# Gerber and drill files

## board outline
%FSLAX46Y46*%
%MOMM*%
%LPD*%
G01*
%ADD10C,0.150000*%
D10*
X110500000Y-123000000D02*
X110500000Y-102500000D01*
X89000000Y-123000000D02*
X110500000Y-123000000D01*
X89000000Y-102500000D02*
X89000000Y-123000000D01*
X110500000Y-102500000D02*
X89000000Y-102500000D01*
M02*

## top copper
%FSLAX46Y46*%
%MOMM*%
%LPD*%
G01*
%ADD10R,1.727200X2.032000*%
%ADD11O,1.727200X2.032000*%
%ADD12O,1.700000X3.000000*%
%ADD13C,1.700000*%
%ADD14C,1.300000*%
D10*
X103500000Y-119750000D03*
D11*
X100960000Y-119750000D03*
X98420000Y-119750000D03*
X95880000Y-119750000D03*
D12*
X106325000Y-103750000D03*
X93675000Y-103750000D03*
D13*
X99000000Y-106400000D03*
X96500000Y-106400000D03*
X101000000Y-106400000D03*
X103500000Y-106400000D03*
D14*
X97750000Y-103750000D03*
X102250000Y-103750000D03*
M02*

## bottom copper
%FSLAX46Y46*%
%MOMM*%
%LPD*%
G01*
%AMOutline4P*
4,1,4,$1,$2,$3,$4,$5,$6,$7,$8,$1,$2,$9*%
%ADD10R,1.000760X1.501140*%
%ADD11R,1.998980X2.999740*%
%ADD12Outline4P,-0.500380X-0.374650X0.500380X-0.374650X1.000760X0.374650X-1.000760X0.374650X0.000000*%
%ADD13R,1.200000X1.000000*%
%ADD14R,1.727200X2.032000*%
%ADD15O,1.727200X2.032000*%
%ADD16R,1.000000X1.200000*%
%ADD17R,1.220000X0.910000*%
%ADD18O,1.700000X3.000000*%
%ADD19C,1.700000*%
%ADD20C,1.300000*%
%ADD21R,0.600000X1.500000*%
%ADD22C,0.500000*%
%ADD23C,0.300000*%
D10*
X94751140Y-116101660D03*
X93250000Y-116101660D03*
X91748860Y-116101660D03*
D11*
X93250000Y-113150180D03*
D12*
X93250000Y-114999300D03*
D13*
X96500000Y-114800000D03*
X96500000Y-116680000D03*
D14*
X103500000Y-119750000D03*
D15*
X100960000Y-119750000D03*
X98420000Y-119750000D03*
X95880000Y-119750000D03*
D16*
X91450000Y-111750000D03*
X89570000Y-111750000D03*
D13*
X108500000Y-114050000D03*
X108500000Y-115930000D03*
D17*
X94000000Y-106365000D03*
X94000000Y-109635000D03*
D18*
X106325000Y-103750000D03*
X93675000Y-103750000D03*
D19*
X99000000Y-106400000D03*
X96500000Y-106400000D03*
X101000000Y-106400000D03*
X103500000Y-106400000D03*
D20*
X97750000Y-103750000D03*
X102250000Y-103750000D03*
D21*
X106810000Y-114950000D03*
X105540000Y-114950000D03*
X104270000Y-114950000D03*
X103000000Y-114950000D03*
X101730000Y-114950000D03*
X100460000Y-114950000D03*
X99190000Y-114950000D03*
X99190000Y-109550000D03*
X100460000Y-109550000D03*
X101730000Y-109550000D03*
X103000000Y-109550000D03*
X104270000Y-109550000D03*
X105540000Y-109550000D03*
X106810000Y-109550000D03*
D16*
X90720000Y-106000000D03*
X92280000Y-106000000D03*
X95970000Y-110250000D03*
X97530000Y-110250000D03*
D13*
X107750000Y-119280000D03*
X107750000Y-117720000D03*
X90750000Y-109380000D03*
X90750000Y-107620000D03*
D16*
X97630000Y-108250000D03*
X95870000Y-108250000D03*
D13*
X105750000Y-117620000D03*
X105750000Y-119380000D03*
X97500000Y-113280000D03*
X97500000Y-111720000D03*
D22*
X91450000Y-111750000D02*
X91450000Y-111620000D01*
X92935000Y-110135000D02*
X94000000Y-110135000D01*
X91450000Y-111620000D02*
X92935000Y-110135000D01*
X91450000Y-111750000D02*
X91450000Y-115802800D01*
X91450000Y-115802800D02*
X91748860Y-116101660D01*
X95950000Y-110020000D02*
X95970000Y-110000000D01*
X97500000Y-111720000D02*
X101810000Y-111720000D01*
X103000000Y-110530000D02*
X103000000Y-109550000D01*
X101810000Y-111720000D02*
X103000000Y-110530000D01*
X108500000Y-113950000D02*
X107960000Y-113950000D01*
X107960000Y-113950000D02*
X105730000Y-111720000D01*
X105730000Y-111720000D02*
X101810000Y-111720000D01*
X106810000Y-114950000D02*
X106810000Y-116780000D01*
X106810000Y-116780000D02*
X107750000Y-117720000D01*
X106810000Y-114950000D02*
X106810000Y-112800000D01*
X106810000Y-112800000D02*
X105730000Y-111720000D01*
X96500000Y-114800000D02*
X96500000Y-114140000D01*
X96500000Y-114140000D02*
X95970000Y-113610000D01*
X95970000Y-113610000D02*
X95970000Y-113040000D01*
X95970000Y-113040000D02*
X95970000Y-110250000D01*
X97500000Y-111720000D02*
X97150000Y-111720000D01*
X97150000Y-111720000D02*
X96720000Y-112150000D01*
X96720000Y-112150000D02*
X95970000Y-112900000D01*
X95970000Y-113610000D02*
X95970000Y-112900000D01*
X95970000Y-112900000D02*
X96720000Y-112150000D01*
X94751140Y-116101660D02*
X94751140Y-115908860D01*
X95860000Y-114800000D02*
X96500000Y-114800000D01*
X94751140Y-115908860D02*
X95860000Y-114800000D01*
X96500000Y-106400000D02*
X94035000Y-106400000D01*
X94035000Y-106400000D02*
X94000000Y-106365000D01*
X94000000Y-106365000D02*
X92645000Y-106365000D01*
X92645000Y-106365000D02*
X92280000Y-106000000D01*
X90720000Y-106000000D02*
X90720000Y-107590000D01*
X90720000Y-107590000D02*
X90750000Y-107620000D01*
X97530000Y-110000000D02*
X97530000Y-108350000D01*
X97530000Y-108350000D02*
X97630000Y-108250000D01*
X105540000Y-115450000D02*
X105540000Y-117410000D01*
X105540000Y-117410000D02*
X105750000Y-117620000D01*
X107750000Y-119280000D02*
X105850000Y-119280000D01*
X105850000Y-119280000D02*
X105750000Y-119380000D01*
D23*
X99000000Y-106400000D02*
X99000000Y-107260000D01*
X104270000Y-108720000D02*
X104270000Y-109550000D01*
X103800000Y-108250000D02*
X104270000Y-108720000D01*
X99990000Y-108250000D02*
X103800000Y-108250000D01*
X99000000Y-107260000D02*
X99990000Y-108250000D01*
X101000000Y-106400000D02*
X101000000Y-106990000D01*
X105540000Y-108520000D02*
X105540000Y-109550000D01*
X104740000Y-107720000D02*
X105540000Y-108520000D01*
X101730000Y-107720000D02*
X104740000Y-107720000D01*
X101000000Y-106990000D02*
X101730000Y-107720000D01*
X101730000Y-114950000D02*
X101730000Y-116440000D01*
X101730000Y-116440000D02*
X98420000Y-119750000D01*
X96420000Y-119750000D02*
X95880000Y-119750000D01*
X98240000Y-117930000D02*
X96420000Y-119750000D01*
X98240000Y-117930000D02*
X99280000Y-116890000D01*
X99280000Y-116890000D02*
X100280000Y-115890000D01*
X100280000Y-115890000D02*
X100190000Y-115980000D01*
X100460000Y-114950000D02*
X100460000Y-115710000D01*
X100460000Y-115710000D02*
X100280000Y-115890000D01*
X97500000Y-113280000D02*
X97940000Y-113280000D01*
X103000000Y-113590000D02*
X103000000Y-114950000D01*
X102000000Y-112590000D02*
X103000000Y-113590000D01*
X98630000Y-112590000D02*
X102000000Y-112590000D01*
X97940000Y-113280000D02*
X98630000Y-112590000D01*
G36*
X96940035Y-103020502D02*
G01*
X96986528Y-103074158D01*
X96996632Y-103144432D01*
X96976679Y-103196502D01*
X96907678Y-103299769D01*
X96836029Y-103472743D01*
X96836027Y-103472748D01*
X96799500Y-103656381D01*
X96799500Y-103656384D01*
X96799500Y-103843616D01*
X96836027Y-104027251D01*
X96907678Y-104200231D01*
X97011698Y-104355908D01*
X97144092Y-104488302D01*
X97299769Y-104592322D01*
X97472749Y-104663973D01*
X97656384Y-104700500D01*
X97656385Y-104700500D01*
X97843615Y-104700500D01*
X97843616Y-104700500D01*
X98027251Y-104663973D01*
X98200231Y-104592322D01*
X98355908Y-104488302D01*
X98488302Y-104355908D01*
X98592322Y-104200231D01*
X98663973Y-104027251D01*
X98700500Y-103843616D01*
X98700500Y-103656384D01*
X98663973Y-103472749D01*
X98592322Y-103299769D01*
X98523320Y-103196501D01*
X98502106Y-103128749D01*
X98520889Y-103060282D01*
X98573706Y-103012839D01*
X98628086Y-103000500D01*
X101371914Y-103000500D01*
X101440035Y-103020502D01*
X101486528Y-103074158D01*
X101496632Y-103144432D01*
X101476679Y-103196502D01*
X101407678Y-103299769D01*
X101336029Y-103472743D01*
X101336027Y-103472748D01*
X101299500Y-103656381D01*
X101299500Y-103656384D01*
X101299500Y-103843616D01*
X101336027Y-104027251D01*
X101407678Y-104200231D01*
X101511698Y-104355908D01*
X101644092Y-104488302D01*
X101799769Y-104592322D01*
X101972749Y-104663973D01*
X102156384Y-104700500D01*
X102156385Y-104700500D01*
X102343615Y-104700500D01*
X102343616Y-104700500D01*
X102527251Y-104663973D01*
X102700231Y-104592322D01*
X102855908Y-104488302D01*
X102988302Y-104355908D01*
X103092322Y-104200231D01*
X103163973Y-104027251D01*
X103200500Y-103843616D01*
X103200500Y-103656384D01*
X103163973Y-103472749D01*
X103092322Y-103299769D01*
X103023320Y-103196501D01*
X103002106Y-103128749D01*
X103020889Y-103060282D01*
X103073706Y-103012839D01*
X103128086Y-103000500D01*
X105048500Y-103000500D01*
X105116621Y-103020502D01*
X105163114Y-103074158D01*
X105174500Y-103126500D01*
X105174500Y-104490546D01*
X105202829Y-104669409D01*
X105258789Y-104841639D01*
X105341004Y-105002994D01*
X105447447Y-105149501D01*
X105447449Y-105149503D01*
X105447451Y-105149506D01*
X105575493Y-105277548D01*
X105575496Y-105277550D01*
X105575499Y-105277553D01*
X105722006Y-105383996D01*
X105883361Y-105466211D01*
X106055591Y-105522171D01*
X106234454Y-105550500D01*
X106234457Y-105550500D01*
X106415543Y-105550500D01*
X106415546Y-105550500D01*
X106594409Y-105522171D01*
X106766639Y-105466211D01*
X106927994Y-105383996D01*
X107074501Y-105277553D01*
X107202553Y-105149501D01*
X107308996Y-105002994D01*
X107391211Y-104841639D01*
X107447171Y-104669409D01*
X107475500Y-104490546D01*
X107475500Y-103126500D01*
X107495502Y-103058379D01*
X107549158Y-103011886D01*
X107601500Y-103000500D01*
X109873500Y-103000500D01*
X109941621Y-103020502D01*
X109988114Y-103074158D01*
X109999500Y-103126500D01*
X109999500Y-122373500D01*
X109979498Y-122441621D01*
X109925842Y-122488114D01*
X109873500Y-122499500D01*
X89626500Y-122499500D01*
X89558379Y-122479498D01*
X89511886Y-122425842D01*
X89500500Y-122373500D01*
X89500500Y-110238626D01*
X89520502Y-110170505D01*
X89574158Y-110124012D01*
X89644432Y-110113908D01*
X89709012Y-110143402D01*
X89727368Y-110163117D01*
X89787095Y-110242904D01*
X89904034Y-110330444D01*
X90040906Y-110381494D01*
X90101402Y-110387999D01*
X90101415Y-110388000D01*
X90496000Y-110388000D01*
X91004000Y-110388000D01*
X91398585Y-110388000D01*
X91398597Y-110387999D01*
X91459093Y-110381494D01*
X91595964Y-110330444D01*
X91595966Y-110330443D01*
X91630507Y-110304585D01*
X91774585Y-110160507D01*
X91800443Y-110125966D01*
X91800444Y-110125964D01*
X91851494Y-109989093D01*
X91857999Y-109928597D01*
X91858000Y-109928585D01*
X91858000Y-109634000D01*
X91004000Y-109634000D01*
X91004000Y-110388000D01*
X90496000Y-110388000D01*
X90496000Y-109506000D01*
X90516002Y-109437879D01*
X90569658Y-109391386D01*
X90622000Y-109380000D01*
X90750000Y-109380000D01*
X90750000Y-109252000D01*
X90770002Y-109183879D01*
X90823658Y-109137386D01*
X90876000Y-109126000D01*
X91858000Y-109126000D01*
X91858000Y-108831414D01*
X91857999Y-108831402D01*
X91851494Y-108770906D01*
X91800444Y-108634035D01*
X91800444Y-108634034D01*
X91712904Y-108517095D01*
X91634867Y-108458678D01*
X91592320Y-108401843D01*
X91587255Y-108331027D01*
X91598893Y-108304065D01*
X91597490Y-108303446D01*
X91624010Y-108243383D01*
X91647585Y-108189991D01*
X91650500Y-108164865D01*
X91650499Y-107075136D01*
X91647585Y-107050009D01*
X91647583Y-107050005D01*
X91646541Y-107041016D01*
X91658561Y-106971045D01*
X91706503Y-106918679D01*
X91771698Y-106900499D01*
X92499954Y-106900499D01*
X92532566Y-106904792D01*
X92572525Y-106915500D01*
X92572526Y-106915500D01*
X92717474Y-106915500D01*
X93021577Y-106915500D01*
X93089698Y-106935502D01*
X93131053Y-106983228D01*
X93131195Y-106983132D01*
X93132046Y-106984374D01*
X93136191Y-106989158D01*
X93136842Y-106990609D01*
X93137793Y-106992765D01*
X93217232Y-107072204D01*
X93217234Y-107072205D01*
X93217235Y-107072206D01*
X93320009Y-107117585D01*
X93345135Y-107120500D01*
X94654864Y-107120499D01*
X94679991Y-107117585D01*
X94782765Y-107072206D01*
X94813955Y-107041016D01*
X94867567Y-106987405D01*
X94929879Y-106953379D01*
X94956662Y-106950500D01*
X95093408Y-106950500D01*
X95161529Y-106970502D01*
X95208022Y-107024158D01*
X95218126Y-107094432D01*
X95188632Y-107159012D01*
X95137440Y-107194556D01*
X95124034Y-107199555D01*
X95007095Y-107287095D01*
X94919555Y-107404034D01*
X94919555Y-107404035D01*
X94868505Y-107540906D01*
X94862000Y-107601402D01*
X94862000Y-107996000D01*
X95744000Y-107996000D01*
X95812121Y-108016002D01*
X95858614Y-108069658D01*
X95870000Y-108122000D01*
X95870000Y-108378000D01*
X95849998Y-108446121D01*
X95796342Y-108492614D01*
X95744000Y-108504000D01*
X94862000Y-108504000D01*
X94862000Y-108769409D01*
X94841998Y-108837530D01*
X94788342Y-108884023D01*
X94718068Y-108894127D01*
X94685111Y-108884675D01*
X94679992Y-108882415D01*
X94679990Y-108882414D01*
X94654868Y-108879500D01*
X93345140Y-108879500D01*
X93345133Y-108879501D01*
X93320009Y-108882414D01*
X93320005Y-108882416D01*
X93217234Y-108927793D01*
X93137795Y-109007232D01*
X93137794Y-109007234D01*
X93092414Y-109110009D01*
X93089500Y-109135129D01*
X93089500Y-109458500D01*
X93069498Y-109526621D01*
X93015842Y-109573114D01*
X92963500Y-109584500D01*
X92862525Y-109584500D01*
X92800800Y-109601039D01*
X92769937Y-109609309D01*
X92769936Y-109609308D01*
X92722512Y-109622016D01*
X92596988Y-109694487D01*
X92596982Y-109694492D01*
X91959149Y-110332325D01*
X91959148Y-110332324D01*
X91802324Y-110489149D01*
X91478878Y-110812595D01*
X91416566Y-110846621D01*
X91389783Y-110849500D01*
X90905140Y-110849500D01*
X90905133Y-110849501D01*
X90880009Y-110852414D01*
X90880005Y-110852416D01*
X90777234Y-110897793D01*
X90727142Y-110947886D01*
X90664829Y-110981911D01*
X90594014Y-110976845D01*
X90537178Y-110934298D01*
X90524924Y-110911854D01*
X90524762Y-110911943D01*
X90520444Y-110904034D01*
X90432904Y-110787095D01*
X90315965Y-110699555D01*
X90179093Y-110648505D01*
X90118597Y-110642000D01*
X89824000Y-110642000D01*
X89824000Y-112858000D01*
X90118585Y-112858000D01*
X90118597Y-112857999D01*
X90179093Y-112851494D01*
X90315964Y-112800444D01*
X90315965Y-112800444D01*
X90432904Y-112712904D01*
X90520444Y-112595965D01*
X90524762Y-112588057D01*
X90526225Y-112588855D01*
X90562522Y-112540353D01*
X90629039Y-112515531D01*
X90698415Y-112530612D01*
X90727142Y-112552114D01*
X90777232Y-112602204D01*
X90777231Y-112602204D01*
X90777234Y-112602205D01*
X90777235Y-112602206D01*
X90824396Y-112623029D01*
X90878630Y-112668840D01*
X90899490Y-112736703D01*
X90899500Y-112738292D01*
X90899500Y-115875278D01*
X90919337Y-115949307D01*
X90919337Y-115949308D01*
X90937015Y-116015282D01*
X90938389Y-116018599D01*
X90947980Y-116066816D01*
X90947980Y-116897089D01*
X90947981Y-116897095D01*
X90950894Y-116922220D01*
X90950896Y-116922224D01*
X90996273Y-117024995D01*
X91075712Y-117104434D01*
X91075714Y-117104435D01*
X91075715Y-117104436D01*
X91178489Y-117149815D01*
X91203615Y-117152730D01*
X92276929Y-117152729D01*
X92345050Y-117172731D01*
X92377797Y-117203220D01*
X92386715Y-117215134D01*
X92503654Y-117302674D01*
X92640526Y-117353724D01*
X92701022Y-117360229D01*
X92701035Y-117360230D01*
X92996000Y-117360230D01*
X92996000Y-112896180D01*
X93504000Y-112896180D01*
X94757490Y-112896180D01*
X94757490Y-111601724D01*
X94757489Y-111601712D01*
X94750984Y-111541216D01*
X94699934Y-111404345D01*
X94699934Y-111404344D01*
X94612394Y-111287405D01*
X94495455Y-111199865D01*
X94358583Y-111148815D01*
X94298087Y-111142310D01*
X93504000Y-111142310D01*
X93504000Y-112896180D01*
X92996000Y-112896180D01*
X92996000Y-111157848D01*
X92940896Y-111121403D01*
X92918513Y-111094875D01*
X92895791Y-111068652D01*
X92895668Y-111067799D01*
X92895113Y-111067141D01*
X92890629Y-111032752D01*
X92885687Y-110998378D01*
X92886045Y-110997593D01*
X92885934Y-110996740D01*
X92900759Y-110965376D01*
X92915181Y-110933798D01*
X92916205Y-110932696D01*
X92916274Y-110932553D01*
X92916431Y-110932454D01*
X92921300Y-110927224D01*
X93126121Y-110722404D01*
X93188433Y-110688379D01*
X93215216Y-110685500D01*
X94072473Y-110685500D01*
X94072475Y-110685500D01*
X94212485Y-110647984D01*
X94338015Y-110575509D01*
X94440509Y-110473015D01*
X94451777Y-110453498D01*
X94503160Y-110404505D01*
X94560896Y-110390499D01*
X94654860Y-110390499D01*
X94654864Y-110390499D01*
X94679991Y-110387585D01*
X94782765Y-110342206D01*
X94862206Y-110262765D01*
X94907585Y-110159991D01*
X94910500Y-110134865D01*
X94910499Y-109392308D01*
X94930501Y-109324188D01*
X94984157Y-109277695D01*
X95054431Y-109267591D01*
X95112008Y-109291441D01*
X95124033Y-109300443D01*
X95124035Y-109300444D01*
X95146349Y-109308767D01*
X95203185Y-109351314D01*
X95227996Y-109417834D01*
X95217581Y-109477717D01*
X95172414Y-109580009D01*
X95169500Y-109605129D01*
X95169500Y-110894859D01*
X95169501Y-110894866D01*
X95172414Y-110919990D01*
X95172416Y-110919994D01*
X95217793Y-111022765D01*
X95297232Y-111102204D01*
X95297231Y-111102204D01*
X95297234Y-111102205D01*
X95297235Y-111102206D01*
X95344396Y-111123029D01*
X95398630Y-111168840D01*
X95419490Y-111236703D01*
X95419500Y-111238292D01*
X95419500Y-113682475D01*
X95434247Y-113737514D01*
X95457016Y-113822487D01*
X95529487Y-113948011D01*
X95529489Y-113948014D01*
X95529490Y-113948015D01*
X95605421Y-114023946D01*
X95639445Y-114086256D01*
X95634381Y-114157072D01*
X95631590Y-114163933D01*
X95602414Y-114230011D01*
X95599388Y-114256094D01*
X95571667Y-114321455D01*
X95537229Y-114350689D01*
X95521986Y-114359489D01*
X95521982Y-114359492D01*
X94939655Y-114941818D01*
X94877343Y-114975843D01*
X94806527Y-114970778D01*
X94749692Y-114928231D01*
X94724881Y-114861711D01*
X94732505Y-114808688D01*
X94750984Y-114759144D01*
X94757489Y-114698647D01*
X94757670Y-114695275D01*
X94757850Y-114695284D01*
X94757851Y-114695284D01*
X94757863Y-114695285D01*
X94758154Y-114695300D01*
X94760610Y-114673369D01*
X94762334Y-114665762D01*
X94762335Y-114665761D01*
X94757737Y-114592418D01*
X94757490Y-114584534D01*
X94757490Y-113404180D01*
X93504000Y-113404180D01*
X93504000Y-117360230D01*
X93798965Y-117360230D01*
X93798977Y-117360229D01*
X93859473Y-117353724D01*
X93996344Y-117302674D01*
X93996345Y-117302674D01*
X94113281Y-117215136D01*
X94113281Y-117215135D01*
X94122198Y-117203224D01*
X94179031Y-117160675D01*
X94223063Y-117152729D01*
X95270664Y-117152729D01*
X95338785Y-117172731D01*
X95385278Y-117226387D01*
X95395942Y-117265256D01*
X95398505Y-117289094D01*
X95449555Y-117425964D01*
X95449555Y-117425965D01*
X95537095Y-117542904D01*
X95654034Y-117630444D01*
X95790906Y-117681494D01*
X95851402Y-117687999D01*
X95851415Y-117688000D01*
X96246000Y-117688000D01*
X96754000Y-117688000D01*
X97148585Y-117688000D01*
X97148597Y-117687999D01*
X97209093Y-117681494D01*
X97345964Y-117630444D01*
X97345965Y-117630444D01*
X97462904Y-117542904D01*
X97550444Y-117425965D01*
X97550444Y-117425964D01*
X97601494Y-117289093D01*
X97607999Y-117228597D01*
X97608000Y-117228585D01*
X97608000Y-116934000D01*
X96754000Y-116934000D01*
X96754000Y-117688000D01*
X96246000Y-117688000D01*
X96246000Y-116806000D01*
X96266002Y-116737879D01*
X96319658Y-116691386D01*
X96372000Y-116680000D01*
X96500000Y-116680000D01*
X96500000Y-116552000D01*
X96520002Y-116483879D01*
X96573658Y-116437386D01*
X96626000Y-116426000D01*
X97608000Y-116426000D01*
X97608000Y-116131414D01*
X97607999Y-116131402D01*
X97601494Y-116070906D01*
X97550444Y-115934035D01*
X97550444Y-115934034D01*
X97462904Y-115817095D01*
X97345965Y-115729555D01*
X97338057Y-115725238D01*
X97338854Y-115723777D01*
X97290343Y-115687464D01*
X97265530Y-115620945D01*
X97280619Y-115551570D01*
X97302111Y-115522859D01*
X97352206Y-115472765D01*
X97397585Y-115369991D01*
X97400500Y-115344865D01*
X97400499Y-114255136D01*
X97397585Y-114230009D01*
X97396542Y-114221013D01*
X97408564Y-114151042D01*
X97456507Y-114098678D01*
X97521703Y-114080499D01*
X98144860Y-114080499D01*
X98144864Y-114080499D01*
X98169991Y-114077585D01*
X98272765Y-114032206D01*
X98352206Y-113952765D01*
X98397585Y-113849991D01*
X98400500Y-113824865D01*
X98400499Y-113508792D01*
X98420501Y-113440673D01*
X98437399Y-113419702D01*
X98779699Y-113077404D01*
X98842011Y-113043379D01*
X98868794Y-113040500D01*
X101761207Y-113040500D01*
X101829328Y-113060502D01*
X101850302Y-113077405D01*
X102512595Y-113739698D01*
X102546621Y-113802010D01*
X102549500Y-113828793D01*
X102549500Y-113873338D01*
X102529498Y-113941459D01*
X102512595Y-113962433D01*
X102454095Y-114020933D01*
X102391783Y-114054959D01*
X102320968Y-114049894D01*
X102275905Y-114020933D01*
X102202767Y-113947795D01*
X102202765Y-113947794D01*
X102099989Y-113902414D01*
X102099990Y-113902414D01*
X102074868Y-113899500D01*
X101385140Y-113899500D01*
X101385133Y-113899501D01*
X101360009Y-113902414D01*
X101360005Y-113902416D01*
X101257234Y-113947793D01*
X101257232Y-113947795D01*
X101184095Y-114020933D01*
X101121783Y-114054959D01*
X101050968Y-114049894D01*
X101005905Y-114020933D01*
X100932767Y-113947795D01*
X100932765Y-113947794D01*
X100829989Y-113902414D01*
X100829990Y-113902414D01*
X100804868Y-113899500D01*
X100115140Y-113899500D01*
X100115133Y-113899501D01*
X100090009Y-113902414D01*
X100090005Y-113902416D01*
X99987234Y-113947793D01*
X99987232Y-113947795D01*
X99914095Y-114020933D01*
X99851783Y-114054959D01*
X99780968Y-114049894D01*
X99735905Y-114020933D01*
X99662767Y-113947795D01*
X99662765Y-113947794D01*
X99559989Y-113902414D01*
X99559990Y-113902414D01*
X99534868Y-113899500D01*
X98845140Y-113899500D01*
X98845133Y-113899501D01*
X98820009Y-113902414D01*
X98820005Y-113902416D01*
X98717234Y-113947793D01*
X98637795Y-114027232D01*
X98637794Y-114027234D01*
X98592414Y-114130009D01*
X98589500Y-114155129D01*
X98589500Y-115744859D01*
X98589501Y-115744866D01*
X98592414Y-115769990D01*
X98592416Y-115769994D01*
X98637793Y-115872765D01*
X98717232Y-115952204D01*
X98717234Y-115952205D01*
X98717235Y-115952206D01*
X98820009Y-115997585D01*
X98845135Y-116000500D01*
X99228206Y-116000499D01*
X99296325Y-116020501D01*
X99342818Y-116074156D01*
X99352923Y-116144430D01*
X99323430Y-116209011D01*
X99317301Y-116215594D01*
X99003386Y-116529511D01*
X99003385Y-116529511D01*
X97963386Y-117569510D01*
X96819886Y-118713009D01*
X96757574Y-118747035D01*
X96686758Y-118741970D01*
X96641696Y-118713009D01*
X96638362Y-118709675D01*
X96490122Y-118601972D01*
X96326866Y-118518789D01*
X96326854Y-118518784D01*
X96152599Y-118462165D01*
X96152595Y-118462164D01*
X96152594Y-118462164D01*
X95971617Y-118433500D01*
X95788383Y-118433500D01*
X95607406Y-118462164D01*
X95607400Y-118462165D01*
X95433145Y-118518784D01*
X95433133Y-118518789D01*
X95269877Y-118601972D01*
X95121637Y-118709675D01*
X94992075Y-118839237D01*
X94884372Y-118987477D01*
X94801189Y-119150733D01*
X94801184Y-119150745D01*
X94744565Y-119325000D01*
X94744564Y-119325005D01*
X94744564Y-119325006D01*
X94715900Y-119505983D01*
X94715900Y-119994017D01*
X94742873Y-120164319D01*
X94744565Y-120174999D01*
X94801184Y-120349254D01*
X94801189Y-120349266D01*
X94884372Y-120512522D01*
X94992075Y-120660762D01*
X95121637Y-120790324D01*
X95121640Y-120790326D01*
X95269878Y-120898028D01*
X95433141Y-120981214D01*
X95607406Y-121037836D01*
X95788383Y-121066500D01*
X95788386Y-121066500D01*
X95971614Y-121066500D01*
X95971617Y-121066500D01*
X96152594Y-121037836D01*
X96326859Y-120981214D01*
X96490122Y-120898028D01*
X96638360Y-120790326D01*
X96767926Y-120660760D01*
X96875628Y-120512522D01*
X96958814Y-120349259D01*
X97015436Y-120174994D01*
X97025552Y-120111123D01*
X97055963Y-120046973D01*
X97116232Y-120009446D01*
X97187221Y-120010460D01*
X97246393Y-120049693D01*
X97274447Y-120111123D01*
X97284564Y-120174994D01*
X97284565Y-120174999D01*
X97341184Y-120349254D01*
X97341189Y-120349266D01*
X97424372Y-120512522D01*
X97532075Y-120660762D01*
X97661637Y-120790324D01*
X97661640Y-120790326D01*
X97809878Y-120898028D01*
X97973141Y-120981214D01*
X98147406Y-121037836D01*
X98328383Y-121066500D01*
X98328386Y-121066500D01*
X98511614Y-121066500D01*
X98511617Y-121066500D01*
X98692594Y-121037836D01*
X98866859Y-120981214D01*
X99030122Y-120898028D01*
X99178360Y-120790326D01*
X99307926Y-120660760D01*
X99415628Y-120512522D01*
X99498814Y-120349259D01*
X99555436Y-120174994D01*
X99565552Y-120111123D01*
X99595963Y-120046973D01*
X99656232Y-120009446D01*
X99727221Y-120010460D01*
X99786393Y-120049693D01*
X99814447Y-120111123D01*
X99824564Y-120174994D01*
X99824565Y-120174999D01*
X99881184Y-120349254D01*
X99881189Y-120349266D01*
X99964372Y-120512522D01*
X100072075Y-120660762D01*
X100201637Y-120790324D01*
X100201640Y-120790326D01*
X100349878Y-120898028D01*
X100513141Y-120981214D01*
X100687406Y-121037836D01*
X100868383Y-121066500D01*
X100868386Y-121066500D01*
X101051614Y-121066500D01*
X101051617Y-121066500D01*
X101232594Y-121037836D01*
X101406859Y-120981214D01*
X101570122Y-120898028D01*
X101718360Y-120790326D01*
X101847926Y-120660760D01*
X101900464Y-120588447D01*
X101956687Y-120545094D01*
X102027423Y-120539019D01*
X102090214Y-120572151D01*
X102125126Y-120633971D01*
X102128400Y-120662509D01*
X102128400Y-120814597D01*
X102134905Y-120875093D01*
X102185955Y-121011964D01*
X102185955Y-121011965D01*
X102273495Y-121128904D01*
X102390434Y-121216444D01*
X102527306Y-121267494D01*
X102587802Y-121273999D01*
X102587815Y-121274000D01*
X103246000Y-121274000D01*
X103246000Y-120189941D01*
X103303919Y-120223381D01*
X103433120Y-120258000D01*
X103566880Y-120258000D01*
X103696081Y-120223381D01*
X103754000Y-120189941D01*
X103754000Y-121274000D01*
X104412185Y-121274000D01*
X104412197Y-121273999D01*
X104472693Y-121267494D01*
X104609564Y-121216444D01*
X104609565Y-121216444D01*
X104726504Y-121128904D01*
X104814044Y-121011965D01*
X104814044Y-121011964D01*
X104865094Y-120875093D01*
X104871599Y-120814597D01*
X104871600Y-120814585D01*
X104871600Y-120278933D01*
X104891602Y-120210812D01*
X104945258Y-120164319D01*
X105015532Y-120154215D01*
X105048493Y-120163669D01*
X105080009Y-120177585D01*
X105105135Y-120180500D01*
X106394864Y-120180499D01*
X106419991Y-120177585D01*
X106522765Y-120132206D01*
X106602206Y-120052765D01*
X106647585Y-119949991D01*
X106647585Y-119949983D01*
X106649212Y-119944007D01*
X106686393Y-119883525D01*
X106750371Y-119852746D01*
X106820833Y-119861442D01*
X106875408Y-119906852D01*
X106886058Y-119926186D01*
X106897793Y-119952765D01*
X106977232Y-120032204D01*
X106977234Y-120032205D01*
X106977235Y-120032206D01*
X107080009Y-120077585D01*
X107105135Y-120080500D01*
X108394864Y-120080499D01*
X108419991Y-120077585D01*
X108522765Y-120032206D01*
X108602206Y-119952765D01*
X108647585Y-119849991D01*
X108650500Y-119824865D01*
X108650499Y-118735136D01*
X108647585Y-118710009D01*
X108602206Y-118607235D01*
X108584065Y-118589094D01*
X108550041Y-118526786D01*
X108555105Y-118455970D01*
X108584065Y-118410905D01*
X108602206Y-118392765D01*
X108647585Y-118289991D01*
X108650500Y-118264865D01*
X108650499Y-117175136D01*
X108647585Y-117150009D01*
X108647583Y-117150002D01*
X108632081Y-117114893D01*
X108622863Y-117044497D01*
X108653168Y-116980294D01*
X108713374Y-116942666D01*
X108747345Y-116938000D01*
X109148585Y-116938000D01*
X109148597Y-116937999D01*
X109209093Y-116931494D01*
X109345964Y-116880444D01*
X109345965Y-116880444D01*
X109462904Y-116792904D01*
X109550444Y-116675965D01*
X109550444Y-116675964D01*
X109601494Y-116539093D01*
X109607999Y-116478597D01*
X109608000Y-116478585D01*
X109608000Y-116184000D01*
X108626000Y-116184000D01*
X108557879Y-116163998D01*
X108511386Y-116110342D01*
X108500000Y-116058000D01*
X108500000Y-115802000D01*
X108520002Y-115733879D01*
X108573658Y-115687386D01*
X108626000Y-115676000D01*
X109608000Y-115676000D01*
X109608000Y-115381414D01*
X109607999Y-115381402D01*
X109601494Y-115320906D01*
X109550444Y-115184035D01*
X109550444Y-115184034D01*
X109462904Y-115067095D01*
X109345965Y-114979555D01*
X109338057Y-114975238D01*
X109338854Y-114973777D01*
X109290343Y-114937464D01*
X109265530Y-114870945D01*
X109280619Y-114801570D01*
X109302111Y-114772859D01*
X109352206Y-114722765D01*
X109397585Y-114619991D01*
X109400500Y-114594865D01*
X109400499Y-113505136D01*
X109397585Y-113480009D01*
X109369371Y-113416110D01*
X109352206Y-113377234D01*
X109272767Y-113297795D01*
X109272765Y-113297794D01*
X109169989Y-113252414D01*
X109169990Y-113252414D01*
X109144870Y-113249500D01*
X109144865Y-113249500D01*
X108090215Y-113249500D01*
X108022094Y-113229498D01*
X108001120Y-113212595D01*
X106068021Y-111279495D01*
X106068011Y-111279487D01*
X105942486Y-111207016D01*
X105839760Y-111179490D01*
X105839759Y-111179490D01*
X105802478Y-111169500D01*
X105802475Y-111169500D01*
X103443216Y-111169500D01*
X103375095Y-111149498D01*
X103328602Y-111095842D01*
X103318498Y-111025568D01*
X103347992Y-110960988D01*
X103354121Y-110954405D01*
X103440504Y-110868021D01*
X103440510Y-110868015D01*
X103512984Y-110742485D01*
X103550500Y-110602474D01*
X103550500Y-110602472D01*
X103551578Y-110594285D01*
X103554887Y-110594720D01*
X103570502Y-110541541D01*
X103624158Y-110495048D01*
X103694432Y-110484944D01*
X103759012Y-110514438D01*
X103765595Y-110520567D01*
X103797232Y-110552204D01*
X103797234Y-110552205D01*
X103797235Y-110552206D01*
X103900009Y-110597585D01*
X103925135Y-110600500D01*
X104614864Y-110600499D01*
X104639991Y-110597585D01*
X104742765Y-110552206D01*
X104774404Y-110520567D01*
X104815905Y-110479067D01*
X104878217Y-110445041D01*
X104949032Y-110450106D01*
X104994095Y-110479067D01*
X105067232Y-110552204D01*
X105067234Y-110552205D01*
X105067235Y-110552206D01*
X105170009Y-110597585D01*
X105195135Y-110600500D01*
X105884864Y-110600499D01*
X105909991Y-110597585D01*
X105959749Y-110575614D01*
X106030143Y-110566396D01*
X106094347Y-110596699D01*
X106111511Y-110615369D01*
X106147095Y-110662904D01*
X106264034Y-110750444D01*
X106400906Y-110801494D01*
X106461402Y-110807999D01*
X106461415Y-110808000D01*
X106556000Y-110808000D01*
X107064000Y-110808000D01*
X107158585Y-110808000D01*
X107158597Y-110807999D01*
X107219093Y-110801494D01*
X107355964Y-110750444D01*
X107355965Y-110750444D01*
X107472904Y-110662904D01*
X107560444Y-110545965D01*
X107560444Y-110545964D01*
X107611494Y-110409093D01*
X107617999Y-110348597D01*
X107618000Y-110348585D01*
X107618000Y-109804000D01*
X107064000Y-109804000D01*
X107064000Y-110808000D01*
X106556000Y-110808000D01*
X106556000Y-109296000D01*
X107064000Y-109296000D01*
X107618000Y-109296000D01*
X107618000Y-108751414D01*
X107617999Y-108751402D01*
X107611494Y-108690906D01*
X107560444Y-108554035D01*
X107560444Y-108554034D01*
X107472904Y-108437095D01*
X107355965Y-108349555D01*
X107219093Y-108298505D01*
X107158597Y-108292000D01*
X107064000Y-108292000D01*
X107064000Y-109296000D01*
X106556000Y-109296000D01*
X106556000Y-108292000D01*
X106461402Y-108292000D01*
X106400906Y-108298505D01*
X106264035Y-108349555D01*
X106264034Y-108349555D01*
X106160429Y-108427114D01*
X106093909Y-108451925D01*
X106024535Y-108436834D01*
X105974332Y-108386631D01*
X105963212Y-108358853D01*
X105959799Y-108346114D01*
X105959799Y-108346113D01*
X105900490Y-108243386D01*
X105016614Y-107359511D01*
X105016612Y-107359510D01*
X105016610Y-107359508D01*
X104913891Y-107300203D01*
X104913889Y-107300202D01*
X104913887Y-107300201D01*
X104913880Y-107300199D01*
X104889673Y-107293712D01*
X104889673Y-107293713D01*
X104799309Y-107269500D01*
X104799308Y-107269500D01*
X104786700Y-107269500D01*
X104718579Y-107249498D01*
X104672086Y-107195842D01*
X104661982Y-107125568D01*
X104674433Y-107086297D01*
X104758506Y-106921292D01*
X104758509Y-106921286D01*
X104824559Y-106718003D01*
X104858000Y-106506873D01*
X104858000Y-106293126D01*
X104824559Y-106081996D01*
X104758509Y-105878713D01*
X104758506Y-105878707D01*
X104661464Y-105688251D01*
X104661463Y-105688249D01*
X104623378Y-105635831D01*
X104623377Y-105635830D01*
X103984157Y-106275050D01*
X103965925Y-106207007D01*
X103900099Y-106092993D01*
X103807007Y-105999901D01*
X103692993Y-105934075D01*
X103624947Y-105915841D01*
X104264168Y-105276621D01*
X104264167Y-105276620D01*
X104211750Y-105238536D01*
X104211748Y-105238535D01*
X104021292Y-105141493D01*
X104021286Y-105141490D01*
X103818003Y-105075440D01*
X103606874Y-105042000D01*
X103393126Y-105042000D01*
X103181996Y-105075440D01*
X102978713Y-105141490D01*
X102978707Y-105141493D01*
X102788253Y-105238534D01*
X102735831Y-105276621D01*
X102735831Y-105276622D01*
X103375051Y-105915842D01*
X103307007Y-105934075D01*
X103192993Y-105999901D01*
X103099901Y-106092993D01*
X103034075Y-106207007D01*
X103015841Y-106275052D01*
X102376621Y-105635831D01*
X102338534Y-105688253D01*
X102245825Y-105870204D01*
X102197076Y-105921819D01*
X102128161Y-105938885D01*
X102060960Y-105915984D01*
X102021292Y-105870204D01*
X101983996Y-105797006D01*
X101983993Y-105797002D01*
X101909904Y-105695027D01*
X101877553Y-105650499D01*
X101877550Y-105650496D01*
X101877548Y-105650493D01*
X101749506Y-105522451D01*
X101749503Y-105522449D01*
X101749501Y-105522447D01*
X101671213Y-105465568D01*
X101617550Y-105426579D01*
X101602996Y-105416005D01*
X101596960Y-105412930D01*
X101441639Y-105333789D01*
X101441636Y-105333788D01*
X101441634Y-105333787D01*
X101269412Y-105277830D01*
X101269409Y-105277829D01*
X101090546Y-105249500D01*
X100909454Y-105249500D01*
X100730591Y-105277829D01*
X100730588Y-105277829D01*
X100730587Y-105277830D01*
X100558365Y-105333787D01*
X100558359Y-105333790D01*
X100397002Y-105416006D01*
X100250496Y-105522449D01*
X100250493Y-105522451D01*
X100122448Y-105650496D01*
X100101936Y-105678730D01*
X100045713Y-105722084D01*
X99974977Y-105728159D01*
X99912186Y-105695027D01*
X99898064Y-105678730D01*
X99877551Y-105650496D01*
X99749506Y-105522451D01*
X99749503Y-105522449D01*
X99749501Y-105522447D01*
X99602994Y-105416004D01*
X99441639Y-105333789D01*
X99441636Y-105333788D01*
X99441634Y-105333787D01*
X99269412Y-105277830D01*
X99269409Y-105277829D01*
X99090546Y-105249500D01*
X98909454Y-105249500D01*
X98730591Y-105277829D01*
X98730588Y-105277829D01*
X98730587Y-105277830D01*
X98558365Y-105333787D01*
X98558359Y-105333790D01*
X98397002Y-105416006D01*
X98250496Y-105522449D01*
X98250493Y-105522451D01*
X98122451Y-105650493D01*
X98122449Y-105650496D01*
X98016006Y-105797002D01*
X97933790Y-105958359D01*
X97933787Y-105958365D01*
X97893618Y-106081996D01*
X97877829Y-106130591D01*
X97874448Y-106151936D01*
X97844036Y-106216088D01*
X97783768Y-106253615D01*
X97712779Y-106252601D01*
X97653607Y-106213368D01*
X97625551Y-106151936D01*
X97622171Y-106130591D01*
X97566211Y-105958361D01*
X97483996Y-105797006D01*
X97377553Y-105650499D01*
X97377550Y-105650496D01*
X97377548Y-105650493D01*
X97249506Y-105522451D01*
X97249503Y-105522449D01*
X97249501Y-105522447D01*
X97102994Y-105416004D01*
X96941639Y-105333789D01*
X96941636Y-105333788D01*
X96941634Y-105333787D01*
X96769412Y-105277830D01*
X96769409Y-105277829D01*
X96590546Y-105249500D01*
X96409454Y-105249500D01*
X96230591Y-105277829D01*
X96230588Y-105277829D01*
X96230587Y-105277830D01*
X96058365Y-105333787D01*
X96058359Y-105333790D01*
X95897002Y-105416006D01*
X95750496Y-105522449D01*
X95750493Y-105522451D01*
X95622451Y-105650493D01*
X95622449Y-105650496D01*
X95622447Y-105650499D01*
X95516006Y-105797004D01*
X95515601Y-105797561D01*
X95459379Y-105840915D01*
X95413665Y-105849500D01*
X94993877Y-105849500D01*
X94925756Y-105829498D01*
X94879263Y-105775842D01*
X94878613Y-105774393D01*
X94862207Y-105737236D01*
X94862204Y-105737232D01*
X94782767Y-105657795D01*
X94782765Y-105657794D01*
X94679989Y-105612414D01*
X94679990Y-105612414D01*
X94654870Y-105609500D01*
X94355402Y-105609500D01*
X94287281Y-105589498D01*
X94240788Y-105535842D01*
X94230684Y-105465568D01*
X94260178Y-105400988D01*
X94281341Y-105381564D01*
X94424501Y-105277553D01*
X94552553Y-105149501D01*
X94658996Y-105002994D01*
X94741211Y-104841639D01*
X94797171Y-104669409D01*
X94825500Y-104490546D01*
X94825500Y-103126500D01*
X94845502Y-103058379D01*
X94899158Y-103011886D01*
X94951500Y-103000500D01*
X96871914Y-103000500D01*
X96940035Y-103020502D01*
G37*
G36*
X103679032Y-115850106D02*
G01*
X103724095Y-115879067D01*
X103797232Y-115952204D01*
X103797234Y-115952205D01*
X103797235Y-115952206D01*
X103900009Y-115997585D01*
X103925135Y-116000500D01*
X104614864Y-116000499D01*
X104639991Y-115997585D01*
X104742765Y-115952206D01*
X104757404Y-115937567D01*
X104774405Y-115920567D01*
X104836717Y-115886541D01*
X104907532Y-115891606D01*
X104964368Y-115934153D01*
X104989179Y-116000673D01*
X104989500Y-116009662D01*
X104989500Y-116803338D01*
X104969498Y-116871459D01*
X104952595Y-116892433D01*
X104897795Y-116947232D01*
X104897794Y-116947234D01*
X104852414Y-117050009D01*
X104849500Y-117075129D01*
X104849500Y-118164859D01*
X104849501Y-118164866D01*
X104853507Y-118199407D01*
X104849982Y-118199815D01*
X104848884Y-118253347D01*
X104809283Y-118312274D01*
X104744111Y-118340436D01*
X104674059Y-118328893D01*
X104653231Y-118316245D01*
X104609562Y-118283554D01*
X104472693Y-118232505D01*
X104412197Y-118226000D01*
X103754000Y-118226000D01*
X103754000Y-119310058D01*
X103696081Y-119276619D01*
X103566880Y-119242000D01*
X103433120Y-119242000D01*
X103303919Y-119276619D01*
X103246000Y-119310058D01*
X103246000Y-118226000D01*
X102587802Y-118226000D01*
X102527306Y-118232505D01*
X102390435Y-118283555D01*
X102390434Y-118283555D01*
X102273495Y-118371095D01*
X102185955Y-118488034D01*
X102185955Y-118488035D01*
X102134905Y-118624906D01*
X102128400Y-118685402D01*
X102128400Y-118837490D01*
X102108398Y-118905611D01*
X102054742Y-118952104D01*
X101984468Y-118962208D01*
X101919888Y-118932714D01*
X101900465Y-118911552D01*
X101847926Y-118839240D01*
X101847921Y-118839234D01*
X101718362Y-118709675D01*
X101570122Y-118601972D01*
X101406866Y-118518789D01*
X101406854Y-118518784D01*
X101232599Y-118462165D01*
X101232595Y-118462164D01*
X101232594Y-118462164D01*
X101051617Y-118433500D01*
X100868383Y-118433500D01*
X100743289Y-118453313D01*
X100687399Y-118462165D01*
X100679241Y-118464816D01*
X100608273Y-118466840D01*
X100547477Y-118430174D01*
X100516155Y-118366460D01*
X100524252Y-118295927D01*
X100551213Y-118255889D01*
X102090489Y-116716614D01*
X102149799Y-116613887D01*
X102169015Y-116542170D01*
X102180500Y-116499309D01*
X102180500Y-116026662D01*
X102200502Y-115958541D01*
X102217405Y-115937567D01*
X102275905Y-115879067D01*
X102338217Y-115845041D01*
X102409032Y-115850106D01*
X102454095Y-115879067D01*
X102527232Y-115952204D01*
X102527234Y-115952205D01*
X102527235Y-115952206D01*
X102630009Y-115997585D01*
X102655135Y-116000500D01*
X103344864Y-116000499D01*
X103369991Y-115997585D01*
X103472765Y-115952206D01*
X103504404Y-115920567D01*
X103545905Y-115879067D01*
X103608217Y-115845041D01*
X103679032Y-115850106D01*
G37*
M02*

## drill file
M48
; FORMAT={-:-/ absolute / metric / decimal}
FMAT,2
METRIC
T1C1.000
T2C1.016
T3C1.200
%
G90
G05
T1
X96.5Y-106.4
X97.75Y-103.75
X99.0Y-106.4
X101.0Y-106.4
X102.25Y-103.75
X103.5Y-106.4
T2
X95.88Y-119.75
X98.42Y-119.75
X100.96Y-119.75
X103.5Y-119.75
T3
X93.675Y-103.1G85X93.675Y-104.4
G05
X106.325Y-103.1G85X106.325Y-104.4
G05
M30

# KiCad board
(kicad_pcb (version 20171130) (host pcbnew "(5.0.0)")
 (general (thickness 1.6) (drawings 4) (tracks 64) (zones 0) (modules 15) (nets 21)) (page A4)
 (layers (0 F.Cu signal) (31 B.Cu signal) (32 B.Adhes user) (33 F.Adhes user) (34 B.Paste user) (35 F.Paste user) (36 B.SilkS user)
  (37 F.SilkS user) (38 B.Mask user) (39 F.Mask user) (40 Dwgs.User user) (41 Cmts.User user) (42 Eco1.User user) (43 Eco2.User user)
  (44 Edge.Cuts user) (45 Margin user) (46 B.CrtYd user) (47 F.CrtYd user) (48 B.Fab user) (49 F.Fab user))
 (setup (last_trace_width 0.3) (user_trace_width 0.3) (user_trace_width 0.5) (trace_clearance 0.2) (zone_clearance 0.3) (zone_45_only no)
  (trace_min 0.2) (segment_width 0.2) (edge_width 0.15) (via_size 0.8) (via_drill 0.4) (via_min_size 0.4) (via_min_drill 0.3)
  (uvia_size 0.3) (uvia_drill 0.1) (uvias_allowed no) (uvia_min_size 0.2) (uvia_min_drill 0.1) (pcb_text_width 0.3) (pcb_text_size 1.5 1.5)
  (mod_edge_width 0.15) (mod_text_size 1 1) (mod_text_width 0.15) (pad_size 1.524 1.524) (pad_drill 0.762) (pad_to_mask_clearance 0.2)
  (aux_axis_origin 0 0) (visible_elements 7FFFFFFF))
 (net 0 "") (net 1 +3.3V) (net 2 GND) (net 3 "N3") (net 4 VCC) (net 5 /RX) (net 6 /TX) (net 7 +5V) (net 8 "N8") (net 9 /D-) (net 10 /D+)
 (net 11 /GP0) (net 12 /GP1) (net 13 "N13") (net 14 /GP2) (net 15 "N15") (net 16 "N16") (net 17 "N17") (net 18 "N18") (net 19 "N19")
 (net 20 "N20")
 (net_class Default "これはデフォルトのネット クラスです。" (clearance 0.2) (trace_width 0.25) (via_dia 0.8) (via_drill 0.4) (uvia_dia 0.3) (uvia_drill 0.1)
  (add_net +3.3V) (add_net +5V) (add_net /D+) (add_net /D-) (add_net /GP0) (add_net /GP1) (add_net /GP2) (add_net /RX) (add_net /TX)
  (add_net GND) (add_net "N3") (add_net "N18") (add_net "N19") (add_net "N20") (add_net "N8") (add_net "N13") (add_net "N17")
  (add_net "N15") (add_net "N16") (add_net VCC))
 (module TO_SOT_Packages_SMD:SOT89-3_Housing (layer B.Cu) (at 93.25 114.25 180)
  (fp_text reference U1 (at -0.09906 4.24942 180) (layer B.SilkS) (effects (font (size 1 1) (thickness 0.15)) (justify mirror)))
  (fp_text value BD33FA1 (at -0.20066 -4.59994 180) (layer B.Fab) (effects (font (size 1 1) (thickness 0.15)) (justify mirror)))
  (pad 1 smd rect (at -1.50114 -1.85166 180) (size 1.00076 1.50114) (layers B.Cu B.Paste B.Mask) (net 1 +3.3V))
  (pad 2 smd rect (at 0 -1.85166 180) (size 1.00076 1.50114) (layers B.Cu B.Paste B.Mask) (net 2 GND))
  (pad 3 smd rect (at 1.50114 -1.85166 180) (size 1.00076 1.50114) (layers B.Cu B.Paste B.Mask) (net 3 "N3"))
  (pad 2 smd rect (at 0 1.09982 180) (size 1.99898 2.99974) (layers B.Cu B.Paste B.Mask) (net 2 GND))
  (pad 2 smd trapezoid (at 0 -0.7493) (size 1.50114 0.7493) (rect_delta 0 -0.50038) (layers B.Cu B.Paste B.Mask) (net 2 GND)))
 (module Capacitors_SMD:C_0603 (layer B.Cu) (at 96.5 115.75 270)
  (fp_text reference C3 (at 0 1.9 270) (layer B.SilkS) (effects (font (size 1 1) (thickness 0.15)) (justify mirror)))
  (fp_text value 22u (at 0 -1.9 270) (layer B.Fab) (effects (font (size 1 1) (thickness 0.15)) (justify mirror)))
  (pad 1 smd rect (at -0.95 0 270) (size 1 1.2) (layers B.Cu B.Paste B.Mask) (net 1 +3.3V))
  (pad 2 smd rect (at 0.93 0 270) (size 1 1.2) (layers B.Cu B.Paste B.Mask) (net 2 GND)))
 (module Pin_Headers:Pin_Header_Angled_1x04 (layer F.Cu) (at 103.5 119.75 270)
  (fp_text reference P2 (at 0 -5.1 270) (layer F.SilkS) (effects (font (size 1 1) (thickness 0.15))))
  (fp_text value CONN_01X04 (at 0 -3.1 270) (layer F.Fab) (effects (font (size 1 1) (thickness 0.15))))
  (pad 1 thru_hole rect (at 0 0 270) (size 2.032 1.7272) (drill 1.016) (layers *.Cu *.Mask F.SilkS) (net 2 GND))
  (pad 2 thru_hole oval (at 0 2.54 270) (size 2.032 1.7272) (drill 1.016) (layers *.Cu *.Mask F.SilkS) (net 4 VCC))
  (pad 3 thru_hole oval (at 0 5.08 270) (size 2.032 1.7272) (drill 1.016) (layers *.Cu *.Mask F.SilkS) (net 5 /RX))
  (pad 4 thru_hole oval (at 0 7.62 270) (size 2.032 1.7272) (drill 1.016) (layers *.Cu *.Mask F.SilkS) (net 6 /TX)))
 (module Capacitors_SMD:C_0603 (layer B.Cu) (at 90.5 111.75 180)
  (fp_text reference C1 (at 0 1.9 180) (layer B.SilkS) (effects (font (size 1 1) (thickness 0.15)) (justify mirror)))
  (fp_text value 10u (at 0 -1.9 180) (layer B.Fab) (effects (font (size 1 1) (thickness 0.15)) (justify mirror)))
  (pad 1 smd rect (at -0.95 0 180) (size 1 1.2) (layers B.Cu B.Paste B.Mask) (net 3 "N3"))
  (pad 2 smd rect (at 0.93 0 180) (size 1 1.2) (layers B.Cu B.Paste B.Mask) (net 2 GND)))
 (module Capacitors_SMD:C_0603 (layer B.Cu) (at 108.5 115 270)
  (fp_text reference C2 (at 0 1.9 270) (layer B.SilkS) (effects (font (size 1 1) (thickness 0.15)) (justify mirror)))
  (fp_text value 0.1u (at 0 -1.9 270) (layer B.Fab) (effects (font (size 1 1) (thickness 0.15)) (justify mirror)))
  (pad 1 smd rect (at -0.95 0 270) (size 1 1.2) (layers B.Cu B.Paste B.Mask) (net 1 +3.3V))
  (pad 2 smd rect (at 0.93 0 270) (size 1 1.2) (layers B.Cu B.Paste B.Mask) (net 2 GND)))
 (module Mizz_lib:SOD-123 (layer B.Cu) (at 94 108 270)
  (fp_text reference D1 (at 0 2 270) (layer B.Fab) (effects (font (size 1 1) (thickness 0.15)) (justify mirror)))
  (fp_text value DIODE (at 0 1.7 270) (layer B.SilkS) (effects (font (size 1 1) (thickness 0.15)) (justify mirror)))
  (pad 1 smd rect (at -1.635 0 270) (size 0.91 1.22) (layers B.Cu B.Paste B.Mask) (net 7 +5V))
  (pad 2 smd rect (at 1.635 0 270) (size 0.91 1.22) (layers B.Cu B.Paste B.Mask) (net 3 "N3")))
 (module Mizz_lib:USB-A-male (layer F.Cu) (at 100 105)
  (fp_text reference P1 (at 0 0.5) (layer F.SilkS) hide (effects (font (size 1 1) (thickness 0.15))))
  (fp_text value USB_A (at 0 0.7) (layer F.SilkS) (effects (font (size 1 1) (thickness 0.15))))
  (pad 5 thru_hole oval (at 6.325 -1.25) (size 1.7 3) (drill oval 1.2 2.5) (layers *.Cu *.Mask F.SilkS) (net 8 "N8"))
  (pad 5 thru_hole oval (at -6.325 -1.25) (size 1.7 3) (drill oval 1.2 2.5) (layers *.Cu *.Mask F.SilkS) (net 8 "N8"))
  (pad 2 thru_hole circle (at -1 1.4) (size 1.7 1.7) (drill 1) (layers *.Cu *.Mask F.SilkS) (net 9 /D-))
  (pad 1 thru_hole circle (at -3.5 1.4) (size 1.7 1.7) (drill 1) (layers *.Cu *.Mask F.SilkS) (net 7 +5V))
  (pad 3 thru_hole circle (at 1 1.4) (size 1.7 1.7) (drill 1) (layers *.Cu *.Mask F.SilkS) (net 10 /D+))
  (pad 4 thru_hole circle (at 3.5 1.4) (size 1.7 1.7) (drill 1) (layers *.Cu *.Mask F.SilkS) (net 2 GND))
  (pad "" thru_hole circle (at -2.25 -1.25) (size 1.3 1.3) (drill 1) (layers *.Cu *.Mask F.SilkS))
  (pad "" thru_hole circle (at 2.25 -1.25) (size 1.3 1.3) (drill 1) (layers *.Cu *.Mask F.SilkS)))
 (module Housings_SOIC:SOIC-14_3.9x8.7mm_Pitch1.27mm (layer B.Cu) (at 103 112.25 90)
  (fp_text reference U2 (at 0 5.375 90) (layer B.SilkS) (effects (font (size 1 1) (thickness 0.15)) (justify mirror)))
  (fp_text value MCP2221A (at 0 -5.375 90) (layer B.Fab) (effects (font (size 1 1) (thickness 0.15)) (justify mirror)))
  (pad 1 smd rect (at -2.7 3.81 90) (size 1.5 0.6) (layers B.Cu B.Paste B.Mask) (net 1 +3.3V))
  (pad 2 smd rect (at -2.7 2.54 90) (size 1.5 0.6) (layers B.Cu B.Paste B.Mask) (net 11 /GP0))
  (pad 3 smd rect (at -2.7 1.27 90) (size 1.5 0.6) (layers B.Cu B.Paste B.Mask) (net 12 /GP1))
  (pad 4 smd rect (at -2.7 0 90) (size 1.5 0.6) (layers B.Cu B.Paste B.Mask) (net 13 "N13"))
  (pad 5 smd rect (at -2.7 -1.27 90) (size 1.5 0.6) (layers B.Cu B.Paste B.Mask) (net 5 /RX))
  (pad 6 smd rect (at -2.7 -2.54 90) (size 1.5 0.6) (layers B.Cu B.Paste B.Mask) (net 6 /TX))
  (pad 7 smd rect (at -2.7 -3.81 90) (size 1.5 0.6) (layers B.Cu B.Paste B.Mask) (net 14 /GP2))
  (pad 8 smd rect (at 2.7 -3.81 90) (size 1.5 0.6) (layers B.Cu B.Paste B.Mask) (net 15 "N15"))
  (pad 9 smd rect (at 2.7 -2.54 90) (size 1.5 0.6) (layers B.Cu B.Paste B.Mask) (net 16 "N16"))
  (pad 10 smd rect (at 2.7 -1.27 90) (size 1.5 0.6) (layers B.Cu B.Paste B.Mask) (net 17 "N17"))
  (pad 11 smd rect (at 2.7 0 90) (size 1.5 0.6) (layers B.Cu B.Paste B.Mask) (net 1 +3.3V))
  (pad 12 smd rect (at 2.7 1.27 90) (size 1.5 0.6) (layers B.Cu B.Paste B.Mask) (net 9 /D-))
  (pad 13 smd rect (at 2.7 2.54 90) (size 1.5 0.6) (layers B.Cu B.Paste B.Mask) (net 10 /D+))
  (pad 14 smd rect (at 2.7 3.81 90) (size 1.5 0.6) (layers B.Cu B.Paste B.Mask) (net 2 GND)))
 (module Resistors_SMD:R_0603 (layer B.Cu) (at 91.5 106)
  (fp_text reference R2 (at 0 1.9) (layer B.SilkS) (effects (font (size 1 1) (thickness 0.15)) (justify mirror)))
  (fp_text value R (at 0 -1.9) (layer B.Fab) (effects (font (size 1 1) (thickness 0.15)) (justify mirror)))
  (pad 1 smd rect (at -0.78 0) (size 1 1.2) (layers B.Cu B.Paste B.Mask) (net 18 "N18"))
  (pad 2 smd rect (at 0.78 0) (size 1 1.2) (layers B.Cu B.Paste B.Mask) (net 7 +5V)))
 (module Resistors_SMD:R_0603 (layer B.Cu) (at 96.75 110.25 180)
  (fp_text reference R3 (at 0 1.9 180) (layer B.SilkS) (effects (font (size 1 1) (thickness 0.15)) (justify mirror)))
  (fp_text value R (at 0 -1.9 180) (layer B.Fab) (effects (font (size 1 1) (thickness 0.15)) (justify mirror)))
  (pad 2 smd rect (at 0.78 0 180) (size 1 1.2) (layers B.Cu B.Paste B.Mask) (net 1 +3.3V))
  (pad 1 smd rect (at -0.78 0 180) (size 1 1.2) (layers B.Cu B.Paste B.Mask) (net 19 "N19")))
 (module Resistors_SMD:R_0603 (layer B.Cu) (at 107.75 118.5 90)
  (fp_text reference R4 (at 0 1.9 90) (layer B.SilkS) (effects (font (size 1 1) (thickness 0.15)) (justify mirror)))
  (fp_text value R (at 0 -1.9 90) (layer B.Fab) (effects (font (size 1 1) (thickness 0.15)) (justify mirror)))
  (pad 1 smd rect (at -0.78 0 90) (size 1 1.2) (layers B.Cu B.Paste B.Mask) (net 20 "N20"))
  (pad 2 smd rect (at 0.78 0 90) (size 1 1.2) (layers B.Cu B.Paste B.Mask) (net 1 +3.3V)))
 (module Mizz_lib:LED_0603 (layer B.Cu) (at 90.75 108.5 90)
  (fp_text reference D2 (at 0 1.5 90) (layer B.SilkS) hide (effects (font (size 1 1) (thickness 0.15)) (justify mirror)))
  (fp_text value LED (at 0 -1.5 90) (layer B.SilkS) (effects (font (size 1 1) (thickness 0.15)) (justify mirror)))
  (pad 2 smd rect (at -0.88 0 270) (size 1 1.2) (layers B.Cu B.Paste B.Mask) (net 2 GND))
  (pad 1 smd rect (at 0.88 0 270) (size 1 1.2) (layers B.Cu B.Paste B.Mask) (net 18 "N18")))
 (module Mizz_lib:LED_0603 (layer B.Cu) (at 96.75 108.25)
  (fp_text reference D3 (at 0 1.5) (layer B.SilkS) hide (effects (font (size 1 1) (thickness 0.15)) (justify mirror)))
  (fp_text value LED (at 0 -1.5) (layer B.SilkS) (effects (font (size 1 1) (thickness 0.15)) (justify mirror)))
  (pad 1 smd rect (at 0.88 0 180) (size 1 1.2) (layers B.Cu B.Paste B.Mask) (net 19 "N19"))
  (pad 2 smd rect (at -0.88 0 180) (size 1 1.2) (layers B.Cu B.Paste B.Mask) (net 2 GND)))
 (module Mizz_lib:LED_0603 (layer B.Cu) (at 105.75 118.5 270)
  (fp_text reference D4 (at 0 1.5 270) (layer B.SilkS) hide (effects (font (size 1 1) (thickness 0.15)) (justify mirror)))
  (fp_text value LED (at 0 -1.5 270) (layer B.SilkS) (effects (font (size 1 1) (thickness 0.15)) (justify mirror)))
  (pad 2 smd rect (at -0.88 0 90) (size 1 1.2) (layers B.Cu B.Paste B.Mask) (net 11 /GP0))
  (pad 1 smd rect (at 0.88 0 90) (size 1 1.2) (layers B.Cu B.Paste B.Mask) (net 20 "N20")))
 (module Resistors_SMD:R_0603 (layer B.Cu) (at 97.5 112.5 90)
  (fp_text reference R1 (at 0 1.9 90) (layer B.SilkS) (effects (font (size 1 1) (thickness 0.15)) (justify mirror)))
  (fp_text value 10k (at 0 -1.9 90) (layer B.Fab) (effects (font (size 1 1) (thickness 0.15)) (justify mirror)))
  (pad 1 smd rect (at -0.78 0 90) (size 1 1.2) (layers B.Cu B.Paste B.Mask) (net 13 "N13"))
  (pad 2 smd rect (at 0.78 0 90) (size 1 1.2) (layers B.Cu B.Paste B.Mask) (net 1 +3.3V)))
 (gr_line (start 110.5 123) (end 110.5 102.5) (angle 90) (layer Edge.Cuts) (width 0.15))
 (gr_line (start 89 123) (end 110.5 123) (angle 90) (layer Edge.Cuts) (width 0.15))
 (gr_line (start 89 102.5) (end 89 123) (angle 90) (layer Edge.Cuts) (width 0.15))
 (gr_line (start 110.5 102.5) (end 89 102.5) (angle 90) (layer Edge.Cuts) (width 0.15))
 (segment (start 91.45 111.75) (end 91.45 111.62) (width 0.5) (layer B.Cu) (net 3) (status C00000))
 (segment (start 92.935 110.135) (end 94 110.135) (width 0.5) (layer B.Cu) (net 3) (status 800000))
 (segment (start 91.45 111.62) (end 92.935 110.135) (width 0.5) (layer B.Cu) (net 3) (status 400000))
 (segment (start 91.45 111.75) (end 91.45 115.8028) (width 0.5) (layer B.Cu) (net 3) (status C00000))
 (segment (start 91.45 115.8028) (end 91.74886 116.10166) (width 0.5) (layer B.Cu) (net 3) (status C00000))
 (segment (start 95.95 110.02) (end 95.97 110) (width 0.5) (layer B.Cu) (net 1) (status C00000))
 (segment (start 97.5 111.72) (end 101.81 111.72) (width 0.5) (layer B.Cu) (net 1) (status 400000))
 (segment (start 103 110.53) (end 103 109.55) (width 0.5) (layer B.Cu) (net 1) (status 800000))
 (segment (start 101.81 111.72) (end 103 110.53) (width 0.5) (layer B.Cu) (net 1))
 (segment (start 108.5 113.95) (end 107.96 113.95) (width 0.5) (layer B.Cu) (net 1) (status C00000))
 (segment (start 107.96 113.95) (end 105.73 111.72) (width 0.5) (layer B.Cu) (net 1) (status 400000))
 (segment (start 105.73 111.72) (end 101.81 111.72) (width 0.5) (layer B.Cu) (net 1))
 (segment (start 106.81 114.95) (end 106.81 116.78) (width 0.5) (layer B.Cu) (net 1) (status 400000))
 (segment (start 106.81 116.78) (end 107.75 117.72) (width 0.5) (layer B.Cu) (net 1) (status 800000))
 (segment (start 106.81 114.95) (end 106.81 112.8) (width 0.5) (layer B.Cu) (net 1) (status 400000))
 (segment (start 106.81 112.8) (end 105.73 111.72) (width 0.5) (layer B.Cu) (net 1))
 (segment (start 96.5 114.8) (end 96.5 114.14) (width 0.5) (layer B.Cu) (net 1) (status 400000))
 (segment (start 96.5 114.14) (end 95.97 113.61) (width 0.5) (layer B.Cu) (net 1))
 (segment (start 95.97 113.61) (end 95.97 113.04) (width 0.5) (layer B.Cu) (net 1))
 (segment (start 95.97 113.04) (end 95.97 110.25) (width 0.5) (layer B.Cu) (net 1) (status 800000))
 (segment (start 97.5 111.72) (end 97.15 111.72) (width 0.5) (layer B.Cu) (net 1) (status C00000))
 (segment (start 97.15 111.72) (end 96.72 112.15) (width 0.5) (layer B.Cu) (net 1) (status 400000))
 (segment (start 96.72 112.15) (end 95.97 112.9) (width 0.5) (layer B.Cu) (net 1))
 (segment (start 95.97 113.61) (end 95.97 112.9) (width 0.5) (layer B.Cu) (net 1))
 (segment (start 95.97 112.9) (end 96.72 112.15) (width 0.5) (layer B.Cu) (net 1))
 (segment (start 94.75114 116.10166) (end 94.75114 115.90886) (width 0.5) (layer B.Cu) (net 1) (status C00000))
 (segment (start 95.86 114.8) (end 96.5 114.8) (width 0.5) (layer B.Cu) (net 1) (status 800000))
 (segment (start 94.75114 115.90886) (end 95.86 114.8) (width 0.5) (layer B.Cu) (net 1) (status 400000))
 (segment (start 96.5 106.4) (end 94.035 106.4) (width 0.5) (layer B.Cu) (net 7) (status C00000))
 (segment (start 94.035 106.4) (end 94 106.365) (width 0.5) (layer B.Cu) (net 7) (status C00000))
 (segment (start 94 106.365) (end 92.645 106.365) (width 0.5) (layer B.Cu) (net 7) (status C00000))
 (segment (start 92.645 106.365) (end 92.28 106) (width 0.5) (layer B.Cu) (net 7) (status C00000))
 (segment (start 90.72 106) (end 90.72 107.59) (width 0.5) (layer B.Cu) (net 18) (status C00000))
 (segment (start 90.72 107.59) (end 90.75 107.62) (width 0.5) (layer B.Cu) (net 18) (status C00000))
 (segment (start 97.53 110) (end 97.53 108.35) (width 0.5) (layer B.Cu) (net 19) (status C00000))
 (segment (start 97.53 108.35) (end 97.63 108.25) (width 0.5) (layer B.Cu) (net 19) (status C00000))
 (segment (start 105.54 115.45) (end 105.54 117.41) (width 0.5) (layer B.Cu) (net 11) (status C00000))
 (segment (start 105.54 117.41) (end 105.75 117.62) (width 0.5) (layer B.Cu) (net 11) (status C00000))
 (segment (start 107.75 119.28) (end 105.85 119.28) (width 0.5) (layer B.Cu) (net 20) (status C00000))
 (segment (start 105.85 119.28) (end 105.75 119.38) (width 0.5) (layer B.Cu) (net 20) (status C00000))
 (segment (start 99 106.4) (end 99 107.26) (width 0.3) (layer B.Cu) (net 9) (status 400000))
 (segment (start 104.27 108.72) (end 104.27 109.55) (width 0.3) (layer B.Cu) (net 9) (status 800000))
 (segment (start 103.8 108.25) (end 104.27 108.72) (width 0.3) (layer B.Cu) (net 9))
 (segment (start 99.99 108.25) (end 103.8 108.25) (width 0.3) (layer B.Cu) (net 9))
 (segment (start 99 107.26) (end 99.99 108.25) (width 0.3) (layer B.Cu) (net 9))
 (segment (start 101 106.4) (end 101 106.99) (width 0.3) (layer B.Cu) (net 10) (status C00000))
 (segment (start 105.54 108.52) (end 105.54 109.55) (width 0.3) (layer B.Cu) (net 10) (status 800000))
 (segment (start 104.74 107.72) (end 105.54 108.52) (width 0.3) (layer B.Cu) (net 10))
 (segment (start 101.73 107.72) (end 104.74 107.72) (width 0.3) (layer B.Cu) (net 10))
 (segment (start 101 106.99) (end 101.73 107.72) (width 0.3) (layer B.Cu) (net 10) (status 400000))
 (segment (start 101.73 114.95) (end 101.73 116.44) (width 0.3) (layer B.Cu) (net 5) (status 400000))
 (segment (start 101.73 116.44) (end 98.42 119.75) (width 0.3) (layer B.Cu) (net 5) (status 800000))
 (segment (start 96.42 119.75) (end 95.88 119.75) (width 0.3) (layer B.Cu) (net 6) (status C00000))
 (segment (start 98.24 117.93) (end 96.42 119.75) (width 0.3) (layer B.Cu) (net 6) (status 800000))
 (segment (start 98.24 117.93) (end 99.28 116.89) (width 0.3) (layer B.Cu) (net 6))
 (segment (start 99.28 116.89) (end 100.28 115.89) (width 0.3) (layer B.Cu) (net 6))
 (segment (start 100.28 115.89) (end 100.19 115.98) (width 0.3) (layer B.Cu) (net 6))
 (segment (start 100.46 114.95) (end 100.46 115.71) (width 0.3) (layer B.Cu) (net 6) (status 400000))
 (segment (start 100.46 115.71) (end 100.28 115.89) (width 0.3) (layer B.Cu) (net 6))
 (segment (start 97.5 113.28) (end 97.94 113.28) (width 0.3) (layer B.Cu) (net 13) (status C00000))
 (segment (start 103 113.59) (end 103 114.95) (width 0.3) (layer B.Cu) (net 13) (status 800000))
 (segment (start 102 112.59) (end 103 113.59) (width 0.3) (layer B.Cu) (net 13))
 (segment (start 98.63 112.59) (end 102 112.59) (width 0.3) (layer B.Cu) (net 13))
 (segment (start 97.94 113.28) (end 98.63 112.59) (width 0.3) (layer B.Cu) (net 13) (status 400000))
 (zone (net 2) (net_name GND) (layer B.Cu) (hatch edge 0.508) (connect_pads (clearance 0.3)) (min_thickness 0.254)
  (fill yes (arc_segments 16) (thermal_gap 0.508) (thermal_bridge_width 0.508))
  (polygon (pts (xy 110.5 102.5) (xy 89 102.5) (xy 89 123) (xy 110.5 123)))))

